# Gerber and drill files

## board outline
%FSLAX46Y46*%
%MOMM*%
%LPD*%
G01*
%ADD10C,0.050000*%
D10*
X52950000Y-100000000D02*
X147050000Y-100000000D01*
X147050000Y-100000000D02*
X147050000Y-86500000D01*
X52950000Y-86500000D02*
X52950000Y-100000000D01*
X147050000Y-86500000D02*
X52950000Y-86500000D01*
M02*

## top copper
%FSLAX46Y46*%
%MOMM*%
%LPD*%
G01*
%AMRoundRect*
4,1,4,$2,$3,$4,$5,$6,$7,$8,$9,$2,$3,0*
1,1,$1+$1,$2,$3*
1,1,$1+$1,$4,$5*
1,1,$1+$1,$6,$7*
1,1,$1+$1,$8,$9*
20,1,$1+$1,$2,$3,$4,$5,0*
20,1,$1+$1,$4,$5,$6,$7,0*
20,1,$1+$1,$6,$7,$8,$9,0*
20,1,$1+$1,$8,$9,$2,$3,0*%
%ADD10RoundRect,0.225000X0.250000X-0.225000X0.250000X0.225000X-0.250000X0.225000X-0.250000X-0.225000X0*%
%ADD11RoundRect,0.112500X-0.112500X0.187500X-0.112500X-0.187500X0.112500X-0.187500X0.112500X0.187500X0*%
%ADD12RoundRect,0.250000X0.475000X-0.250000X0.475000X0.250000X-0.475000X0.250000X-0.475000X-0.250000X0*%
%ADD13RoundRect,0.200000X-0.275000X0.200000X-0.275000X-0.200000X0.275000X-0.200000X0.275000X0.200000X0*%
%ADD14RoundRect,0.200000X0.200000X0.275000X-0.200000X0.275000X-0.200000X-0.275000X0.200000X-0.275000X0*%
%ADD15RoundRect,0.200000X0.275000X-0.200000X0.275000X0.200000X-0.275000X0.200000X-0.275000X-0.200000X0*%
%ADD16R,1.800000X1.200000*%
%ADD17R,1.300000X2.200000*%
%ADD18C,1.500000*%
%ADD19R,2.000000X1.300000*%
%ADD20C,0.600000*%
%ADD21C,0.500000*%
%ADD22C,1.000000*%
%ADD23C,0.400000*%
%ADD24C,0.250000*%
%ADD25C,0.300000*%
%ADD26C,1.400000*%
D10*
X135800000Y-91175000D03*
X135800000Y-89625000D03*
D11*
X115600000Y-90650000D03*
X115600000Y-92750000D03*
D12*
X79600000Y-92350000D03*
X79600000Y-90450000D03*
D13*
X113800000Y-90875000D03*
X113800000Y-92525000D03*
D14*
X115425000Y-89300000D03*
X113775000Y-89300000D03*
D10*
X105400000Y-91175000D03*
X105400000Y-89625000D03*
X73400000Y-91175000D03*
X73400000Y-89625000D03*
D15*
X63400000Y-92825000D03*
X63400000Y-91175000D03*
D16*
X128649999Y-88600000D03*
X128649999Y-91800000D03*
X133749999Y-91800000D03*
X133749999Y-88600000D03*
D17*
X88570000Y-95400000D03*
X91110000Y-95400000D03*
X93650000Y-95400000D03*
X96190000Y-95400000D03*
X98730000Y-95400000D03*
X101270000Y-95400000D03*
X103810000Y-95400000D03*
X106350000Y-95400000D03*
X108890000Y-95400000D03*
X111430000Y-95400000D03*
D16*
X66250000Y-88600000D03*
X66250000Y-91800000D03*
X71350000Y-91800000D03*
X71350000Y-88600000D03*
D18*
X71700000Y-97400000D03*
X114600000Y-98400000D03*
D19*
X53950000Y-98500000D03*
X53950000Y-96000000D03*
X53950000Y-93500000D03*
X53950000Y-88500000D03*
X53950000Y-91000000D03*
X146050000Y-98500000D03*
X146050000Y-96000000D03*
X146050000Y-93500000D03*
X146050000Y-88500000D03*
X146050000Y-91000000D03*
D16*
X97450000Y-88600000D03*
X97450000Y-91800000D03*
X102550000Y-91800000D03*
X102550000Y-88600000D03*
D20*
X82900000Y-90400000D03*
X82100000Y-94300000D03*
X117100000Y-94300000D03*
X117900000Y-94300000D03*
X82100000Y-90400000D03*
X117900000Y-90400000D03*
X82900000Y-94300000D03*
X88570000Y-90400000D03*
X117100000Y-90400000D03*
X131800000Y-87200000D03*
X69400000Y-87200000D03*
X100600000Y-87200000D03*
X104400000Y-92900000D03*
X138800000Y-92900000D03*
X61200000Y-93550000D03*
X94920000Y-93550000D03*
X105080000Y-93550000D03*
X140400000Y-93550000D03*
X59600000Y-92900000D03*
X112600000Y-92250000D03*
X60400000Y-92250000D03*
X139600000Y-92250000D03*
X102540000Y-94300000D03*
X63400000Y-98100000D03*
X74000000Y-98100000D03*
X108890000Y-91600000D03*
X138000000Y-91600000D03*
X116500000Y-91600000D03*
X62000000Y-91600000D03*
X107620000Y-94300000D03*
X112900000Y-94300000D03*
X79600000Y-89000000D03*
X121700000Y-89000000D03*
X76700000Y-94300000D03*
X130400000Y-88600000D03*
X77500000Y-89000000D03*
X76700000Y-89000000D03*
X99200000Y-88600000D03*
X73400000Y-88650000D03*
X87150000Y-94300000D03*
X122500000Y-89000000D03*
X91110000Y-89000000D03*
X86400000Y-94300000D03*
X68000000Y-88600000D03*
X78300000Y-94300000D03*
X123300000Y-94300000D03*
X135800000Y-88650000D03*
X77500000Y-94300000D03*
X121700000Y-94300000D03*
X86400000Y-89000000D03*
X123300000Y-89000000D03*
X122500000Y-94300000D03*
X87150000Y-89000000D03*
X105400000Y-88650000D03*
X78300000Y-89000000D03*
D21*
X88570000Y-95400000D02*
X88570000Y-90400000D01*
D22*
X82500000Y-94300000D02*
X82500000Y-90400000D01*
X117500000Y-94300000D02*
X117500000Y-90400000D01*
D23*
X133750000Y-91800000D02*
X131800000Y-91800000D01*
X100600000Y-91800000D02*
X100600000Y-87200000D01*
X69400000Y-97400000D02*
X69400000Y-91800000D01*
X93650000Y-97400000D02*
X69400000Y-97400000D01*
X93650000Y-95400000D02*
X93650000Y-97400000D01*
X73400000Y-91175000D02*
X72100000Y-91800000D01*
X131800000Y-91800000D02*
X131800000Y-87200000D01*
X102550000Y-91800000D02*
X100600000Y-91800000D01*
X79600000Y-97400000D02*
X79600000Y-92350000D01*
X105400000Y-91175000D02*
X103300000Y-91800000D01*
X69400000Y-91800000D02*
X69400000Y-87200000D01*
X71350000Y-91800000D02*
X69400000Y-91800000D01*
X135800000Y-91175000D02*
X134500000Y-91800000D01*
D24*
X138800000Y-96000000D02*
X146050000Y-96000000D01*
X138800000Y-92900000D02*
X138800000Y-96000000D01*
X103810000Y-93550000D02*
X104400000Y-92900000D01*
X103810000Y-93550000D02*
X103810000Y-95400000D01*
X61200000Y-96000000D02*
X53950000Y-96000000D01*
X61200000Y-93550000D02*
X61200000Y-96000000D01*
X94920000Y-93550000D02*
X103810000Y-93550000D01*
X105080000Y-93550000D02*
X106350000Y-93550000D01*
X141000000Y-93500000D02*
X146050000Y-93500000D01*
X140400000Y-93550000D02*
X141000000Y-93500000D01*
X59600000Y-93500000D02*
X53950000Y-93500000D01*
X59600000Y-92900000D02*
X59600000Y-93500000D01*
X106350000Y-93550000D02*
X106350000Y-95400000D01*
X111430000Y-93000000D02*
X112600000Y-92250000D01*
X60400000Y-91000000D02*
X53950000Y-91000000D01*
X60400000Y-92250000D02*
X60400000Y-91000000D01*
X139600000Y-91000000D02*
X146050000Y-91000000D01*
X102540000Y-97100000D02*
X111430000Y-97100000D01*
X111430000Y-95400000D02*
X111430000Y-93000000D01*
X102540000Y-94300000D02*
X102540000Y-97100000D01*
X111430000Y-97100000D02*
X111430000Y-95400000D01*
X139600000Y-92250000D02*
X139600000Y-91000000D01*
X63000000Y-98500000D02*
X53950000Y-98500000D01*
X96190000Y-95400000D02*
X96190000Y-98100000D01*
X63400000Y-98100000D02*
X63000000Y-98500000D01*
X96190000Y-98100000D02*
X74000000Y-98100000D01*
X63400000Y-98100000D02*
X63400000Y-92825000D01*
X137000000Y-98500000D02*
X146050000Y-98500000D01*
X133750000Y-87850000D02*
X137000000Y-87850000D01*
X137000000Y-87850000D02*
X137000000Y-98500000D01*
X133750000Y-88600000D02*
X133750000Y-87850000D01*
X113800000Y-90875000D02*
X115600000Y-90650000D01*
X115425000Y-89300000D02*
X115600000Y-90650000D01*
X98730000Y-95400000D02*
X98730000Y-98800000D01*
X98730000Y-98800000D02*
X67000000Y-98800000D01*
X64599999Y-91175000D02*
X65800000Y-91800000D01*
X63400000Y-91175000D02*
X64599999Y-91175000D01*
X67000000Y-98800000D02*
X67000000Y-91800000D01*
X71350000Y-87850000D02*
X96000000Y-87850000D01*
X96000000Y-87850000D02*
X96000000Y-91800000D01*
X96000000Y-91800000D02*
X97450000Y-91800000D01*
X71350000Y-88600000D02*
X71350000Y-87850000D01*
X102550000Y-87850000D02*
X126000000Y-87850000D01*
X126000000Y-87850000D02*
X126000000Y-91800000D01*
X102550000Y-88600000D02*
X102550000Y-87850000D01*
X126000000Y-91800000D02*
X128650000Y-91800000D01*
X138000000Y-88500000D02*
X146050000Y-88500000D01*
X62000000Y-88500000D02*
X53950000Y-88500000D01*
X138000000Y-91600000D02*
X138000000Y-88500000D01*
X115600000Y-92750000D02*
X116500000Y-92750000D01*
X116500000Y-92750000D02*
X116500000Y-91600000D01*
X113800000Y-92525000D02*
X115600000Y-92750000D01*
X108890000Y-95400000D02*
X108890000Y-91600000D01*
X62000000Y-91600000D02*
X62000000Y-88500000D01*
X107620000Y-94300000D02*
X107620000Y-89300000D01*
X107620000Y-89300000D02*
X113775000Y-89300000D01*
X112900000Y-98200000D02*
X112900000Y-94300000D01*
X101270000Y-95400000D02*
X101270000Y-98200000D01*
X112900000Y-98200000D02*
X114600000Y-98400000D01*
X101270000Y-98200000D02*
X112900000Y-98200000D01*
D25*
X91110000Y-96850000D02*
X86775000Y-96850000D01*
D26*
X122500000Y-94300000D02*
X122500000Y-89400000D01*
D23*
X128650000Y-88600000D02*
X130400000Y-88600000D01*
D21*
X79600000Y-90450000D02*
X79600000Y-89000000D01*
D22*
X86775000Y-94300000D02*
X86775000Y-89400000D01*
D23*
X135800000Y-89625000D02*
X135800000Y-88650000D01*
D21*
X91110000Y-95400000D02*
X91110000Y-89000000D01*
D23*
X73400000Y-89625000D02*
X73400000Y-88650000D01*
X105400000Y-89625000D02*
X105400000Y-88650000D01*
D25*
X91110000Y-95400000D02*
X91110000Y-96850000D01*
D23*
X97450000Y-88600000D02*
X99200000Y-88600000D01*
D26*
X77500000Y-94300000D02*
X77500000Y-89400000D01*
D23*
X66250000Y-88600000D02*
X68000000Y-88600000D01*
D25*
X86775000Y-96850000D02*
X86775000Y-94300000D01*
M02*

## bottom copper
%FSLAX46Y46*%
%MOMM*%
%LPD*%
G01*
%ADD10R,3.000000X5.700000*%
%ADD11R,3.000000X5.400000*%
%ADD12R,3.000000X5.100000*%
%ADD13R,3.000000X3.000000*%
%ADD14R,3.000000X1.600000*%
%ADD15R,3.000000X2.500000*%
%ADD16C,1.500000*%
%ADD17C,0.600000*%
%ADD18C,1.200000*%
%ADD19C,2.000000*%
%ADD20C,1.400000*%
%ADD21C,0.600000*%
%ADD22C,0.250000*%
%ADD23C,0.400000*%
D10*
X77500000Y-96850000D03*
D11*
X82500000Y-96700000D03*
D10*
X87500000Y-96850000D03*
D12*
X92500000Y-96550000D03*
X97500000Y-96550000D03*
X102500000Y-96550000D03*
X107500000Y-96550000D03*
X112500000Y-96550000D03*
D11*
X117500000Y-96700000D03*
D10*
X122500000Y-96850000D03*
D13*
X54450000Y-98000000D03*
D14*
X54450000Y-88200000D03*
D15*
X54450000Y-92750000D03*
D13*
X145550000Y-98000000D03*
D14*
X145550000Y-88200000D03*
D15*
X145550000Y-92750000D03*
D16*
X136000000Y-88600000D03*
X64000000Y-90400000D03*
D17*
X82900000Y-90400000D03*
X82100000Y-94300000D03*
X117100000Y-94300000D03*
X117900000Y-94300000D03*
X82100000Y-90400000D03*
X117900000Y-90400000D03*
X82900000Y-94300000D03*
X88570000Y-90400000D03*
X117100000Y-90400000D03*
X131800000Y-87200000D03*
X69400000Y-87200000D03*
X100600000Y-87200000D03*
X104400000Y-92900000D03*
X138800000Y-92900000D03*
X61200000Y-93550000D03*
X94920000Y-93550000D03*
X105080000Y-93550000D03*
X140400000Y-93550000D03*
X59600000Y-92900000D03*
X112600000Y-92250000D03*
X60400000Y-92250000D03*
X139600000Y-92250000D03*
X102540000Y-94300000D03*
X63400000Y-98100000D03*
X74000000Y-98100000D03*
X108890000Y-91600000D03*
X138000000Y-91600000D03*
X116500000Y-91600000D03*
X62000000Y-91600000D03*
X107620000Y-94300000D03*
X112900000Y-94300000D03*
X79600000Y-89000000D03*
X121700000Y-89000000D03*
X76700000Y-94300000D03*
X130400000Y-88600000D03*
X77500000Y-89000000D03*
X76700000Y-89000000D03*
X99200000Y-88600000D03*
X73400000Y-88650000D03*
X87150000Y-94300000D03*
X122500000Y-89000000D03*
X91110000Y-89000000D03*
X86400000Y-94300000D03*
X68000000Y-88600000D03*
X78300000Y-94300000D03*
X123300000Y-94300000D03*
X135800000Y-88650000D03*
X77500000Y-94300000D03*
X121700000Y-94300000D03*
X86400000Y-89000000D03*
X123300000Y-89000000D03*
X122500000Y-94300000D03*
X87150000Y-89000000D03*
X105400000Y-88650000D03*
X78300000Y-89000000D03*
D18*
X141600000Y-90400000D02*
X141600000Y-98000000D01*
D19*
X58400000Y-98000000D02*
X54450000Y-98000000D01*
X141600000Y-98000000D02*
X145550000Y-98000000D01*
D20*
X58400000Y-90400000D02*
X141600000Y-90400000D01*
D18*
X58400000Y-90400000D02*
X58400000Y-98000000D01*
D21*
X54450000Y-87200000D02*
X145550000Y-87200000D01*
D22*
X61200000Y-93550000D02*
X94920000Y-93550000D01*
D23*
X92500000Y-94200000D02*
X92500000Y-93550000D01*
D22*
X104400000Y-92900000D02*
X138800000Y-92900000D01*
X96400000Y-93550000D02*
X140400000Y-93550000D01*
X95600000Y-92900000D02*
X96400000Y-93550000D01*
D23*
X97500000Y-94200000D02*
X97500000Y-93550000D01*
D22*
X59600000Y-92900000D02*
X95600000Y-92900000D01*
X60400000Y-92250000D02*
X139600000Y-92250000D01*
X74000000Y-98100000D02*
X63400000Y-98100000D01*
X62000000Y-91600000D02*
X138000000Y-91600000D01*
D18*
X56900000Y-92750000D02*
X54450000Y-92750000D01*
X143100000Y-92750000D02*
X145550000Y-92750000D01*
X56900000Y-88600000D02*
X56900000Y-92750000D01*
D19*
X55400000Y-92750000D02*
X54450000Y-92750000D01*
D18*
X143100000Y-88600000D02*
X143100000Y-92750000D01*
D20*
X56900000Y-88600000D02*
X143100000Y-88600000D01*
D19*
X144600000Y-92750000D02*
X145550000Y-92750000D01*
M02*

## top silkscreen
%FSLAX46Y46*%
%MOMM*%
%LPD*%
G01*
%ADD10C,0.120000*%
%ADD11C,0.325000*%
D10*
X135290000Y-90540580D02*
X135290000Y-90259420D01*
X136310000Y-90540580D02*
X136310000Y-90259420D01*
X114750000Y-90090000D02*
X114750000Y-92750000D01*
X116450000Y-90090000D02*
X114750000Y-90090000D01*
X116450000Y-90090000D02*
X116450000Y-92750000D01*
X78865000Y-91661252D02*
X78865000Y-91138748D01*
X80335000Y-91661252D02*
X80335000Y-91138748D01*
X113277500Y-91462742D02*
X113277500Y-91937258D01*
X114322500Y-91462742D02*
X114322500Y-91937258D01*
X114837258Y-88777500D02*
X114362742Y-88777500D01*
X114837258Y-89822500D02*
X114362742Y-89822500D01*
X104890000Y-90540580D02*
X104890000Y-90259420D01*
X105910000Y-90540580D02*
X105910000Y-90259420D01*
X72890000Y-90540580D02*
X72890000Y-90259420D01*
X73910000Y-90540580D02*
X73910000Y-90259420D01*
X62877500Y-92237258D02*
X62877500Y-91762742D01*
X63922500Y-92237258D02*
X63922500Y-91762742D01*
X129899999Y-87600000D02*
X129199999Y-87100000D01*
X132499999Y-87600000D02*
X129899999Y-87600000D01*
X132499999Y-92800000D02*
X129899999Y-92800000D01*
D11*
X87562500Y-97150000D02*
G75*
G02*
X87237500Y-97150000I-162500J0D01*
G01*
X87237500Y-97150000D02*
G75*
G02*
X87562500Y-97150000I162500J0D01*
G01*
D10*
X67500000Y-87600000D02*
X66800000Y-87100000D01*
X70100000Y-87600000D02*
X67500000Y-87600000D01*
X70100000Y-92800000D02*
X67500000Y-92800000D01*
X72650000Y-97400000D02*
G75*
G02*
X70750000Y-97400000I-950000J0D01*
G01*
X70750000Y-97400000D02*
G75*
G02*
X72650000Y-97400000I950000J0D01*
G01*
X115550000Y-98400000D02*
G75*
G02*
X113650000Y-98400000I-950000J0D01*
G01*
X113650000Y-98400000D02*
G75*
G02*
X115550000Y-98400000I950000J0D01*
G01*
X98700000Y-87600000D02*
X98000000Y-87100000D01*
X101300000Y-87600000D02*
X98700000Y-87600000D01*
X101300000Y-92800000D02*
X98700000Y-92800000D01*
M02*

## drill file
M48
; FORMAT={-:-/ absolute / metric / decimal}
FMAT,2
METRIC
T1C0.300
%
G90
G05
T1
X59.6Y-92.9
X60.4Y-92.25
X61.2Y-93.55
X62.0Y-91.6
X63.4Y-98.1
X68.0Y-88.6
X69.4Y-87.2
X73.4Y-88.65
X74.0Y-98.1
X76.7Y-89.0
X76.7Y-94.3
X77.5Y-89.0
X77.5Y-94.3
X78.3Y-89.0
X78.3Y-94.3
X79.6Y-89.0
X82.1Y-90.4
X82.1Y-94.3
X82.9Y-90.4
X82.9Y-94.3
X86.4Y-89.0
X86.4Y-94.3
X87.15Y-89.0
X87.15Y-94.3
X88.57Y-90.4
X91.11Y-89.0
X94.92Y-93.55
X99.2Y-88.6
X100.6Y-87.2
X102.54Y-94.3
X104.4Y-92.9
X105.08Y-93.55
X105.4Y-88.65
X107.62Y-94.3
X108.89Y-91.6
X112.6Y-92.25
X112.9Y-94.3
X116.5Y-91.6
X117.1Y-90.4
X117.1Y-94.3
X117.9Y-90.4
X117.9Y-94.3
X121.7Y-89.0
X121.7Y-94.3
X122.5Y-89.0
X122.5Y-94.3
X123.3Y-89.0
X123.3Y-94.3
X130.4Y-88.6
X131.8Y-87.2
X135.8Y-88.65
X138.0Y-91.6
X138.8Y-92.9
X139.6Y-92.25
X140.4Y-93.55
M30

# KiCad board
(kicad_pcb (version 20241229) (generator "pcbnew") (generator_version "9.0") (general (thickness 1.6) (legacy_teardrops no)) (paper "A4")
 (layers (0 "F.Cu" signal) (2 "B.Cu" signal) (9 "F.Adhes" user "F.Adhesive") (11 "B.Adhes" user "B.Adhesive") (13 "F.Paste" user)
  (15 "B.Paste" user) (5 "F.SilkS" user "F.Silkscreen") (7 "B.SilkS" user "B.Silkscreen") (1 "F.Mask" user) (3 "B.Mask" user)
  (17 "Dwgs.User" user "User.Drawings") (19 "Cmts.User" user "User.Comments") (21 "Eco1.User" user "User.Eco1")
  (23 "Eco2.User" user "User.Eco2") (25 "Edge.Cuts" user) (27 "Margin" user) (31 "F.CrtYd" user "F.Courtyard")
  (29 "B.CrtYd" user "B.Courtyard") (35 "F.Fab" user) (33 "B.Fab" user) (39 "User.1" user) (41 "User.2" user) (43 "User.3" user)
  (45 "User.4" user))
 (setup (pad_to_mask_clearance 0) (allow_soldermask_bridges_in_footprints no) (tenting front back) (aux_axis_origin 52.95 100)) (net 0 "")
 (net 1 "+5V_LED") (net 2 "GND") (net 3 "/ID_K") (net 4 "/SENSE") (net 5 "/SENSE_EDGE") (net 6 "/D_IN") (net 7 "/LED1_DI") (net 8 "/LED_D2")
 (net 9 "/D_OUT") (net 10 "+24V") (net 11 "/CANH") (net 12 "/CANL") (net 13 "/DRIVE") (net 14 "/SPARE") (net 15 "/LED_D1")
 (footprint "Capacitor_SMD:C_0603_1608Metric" (layer "F.Cu") (at 135.8 90.4 90)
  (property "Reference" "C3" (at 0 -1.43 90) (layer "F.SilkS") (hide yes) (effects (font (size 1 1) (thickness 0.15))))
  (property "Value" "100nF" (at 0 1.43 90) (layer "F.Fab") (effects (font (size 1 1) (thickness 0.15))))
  (fp_line (start -0.14058 -0.51) (end 0.14058 -0.51) (stroke (width 0.12) (type solid)) (layer "F.SilkS"))
  (fp_line (start -0.14058 0.51) (end 0.14058 0.51) (stroke (width 0.12) (type solid)) (layer "F.SilkS"))
  (pad "1" smd roundrect (at -0.775 0 90) (size 0.9 0.95) (layers "F.Cu" "F.Mask" "F.Paste") (roundrect_rratio 0.25) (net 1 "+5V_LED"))
  (pad "2" smd roundrect (at 0.775 0 90) (size 0.9 0.95) (layers "F.Cu" "F.Mask" "F.Paste") (roundrect_rratio 0.25) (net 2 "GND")))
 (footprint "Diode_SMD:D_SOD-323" (layer "F.Cu") (at 115.6 91.7 -90)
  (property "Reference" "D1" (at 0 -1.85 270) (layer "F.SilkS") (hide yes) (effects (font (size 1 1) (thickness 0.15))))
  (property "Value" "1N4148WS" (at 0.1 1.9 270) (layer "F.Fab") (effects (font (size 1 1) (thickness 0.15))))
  (fp_line (start -1.61 0.85) (end 1.05 0.85) (stroke (width 0.12) (type solid)) (layer "F.SilkS"))
  (fp_line (start -1.61 -0.85) (end -1.61 0.85) (stroke (width 0.12) (type solid)) (layer "F.SilkS"))
  (fp_line (start -1.61 -0.85) (end 1.05 -0.85) (stroke (width 0.12) (type solid)) (layer "F.SilkS"))
  (pad "1" smd roundrect (at -1.05 0 270) (size 0.6 0.45) (layers "F.Cu" "F.Mask" "F.Paste") (roundrect_rratio 0.25) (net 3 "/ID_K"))
  (pad "2" smd roundrect (at 1.05 0 270) (size 0.6 0.45) (layers "F.Cu" "F.Mask" "F.Paste") (roundrect_rratio 0.25) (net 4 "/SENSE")))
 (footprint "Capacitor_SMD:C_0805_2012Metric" (layer "F.Cu") (at 79.6 91.4 90)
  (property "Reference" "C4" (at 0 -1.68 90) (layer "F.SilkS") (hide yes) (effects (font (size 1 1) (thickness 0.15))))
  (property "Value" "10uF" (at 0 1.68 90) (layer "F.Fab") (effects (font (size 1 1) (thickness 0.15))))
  (fp_line (start -0.261252 -0.735) (end 0.261252 -0.735) (stroke (width 0.12) (type solid)) (layer "F.SilkS"))
  (fp_line (start -0.261252 0.735) (end 0.261252 0.735) (stroke (width 0.12) (type solid)) (layer "F.SilkS"))
  (pad "1" smd roundrect (at -0.95 0 90) (size 1 1.45) (layers "F.Cu" "F.Mask" "F.Paste") (roundrect_rratio 0.25) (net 1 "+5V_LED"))
  (pad "2" smd roundrect (at 0.95 0 90) (size 1 1.45) (layers "F.Cu" "F.Mask" "F.Paste") (roundrect_rratio 0.25) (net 2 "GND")))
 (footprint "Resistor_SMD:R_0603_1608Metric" (layer "F.Cu") (at 113.8 91.7 -90)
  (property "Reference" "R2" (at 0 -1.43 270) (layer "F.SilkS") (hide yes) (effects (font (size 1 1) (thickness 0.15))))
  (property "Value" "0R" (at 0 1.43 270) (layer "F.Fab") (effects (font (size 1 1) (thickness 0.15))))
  (fp_line (start -0.237258 0.5225) (end 0.237258 0.5225) (stroke (width 0.12) (type solid)) (layer "F.SilkS"))
  (fp_line (start -0.237258 -0.5225) (end 0.237258 -0.5225) (stroke (width 0.12) (type solid)) (layer "F.SilkS"))
  (pad "1" smd roundrect (at -0.825 0 270) (size 0.8 0.95) (layers "F.Cu" "F.Mask" "F.Paste") (roundrect_rratio 0.25) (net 3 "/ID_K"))
  (pad "2" smd roundrect (at 0.825 0 270) (size 0.8 0.95) (layers "F.Cu" "F.Mask" "F.Paste") (roundrect_rratio 0.25) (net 4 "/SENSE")))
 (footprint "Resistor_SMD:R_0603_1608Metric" (layer "F.Cu") (at 114.6 89.3 180)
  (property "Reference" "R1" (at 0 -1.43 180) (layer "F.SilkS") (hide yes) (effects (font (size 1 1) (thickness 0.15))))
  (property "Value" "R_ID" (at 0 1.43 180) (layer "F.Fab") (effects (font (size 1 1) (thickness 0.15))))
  (fp_line (start -0.237258 0.5225) (end 0.237258 0.5225) (stroke (width 0.12) (type solid)) (layer "F.SilkS"))
  (fp_line (start -0.237258 -0.5225) (end 0.237258 -0.5225) (stroke (width 0.12) (type solid)) (layer "F.SilkS"))
  (pad "1" smd roundrect (at -0.825 0 180) (size 0.8 0.95) (layers "F.Cu" "F.Mask" "F.Paste") (roundrect_rratio 0.25) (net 3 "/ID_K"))
  (pad "2" smd roundrect (at 0.825 0 180) (size 0.8 0.95) (layers "F.Cu" "F.Mask" "F.Paste") (roundrect_rratio 0.25) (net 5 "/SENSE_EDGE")))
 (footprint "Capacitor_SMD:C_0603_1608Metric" (layer "F.Cu") (at 105.4 90.4 90)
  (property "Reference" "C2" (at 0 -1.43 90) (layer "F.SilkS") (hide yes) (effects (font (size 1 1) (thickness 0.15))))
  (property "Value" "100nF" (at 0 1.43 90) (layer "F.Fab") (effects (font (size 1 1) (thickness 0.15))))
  (fp_line (start -0.14058 -0.51) (end 0.14058 -0.51) (stroke (width 0.12) (type solid)) (layer "F.SilkS"))
  (fp_line (start -0.14058 0.51) (end 0.14058 0.51) (stroke (width 0.12) (type solid)) (layer "F.SilkS"))
  (pad "1" smd roundrect (at -0.775 0 90) (size 0.9 0.95) (layers "F.Cu" "F.Mask" "F.Paste") (roundrect_rratio 0.25) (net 1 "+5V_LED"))
  (pad "2" smd roundrect (at 0.775 0 90) (size 0.9 0.95) (layers "F.Cu" "F.Mask" "F.Paste") (roundrect_rratio 0.25) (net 2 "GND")))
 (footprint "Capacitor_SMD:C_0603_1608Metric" (layer "F.Cu") (at 73.4 90.4 90)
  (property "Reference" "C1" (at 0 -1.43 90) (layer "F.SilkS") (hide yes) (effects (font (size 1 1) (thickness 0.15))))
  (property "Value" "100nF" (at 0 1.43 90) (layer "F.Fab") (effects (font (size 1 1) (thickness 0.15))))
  (fp_line (start -0.14058 -0.51) (end 0.14058 -0.51) (stroke (width 0.12) (type solid)) (layer "F.SilkS"))
  (fp_line (start -0.14058 0.51) (end 0.14058 0.51) (stroke (width 0.12) (type solid)) (layer "F.SilkS"))
  (pad "1" smd roundrect (at -0.775 0 90) (size 0.9 0.95) (layers "F.Cu" "F.Mask" "F.Paste") (roundrect_rratio 0.25) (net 1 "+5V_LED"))
  (pad "2" smd roundrect (at 0.775 0 90) (size 0.9 0.95) (layers "F.Cu" "F.Mask" "F.Paste") (roundrect_rratio 0.25) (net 2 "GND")))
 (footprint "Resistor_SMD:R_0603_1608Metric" (layer "F.Cu") (at 63.4 92 90)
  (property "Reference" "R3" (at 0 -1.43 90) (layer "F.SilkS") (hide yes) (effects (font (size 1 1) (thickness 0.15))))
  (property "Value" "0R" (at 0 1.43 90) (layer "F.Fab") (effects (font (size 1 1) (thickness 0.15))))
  (fp_line (start -0.237258 -0.5225) (end 0.237258 -0.5225) (stroke (width 0.12) (type solid)) (layer "F.SilkS"))
  (fp_line (start -0.237258 0.5225) (end 0.237258 0.5225) (stroke (width 0.12) (type solid)) (layer "F.SilkS"))
  (pad "1" smd roundrect (at -0.825 0 90) (size 0.8 0.95) (layers "F.Cu" "F.Mask" "F.Paste") (roundrect_rratio 0.25) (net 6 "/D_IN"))
  (pad "2" smd roundrect (at 0.825 0 90) (size 0.8 0.95) (layers "F.Cu" "F.Mask" "F.Paste") (roundrect_rratio 0.25) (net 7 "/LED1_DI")))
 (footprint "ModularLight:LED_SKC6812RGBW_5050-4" (layer "F.Cu") (at 131.199999 90.2 180)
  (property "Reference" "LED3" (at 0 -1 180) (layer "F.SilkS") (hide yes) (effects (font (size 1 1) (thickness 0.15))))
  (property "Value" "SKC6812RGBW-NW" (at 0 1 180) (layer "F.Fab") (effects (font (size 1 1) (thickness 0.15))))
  (fp_line (start 1.3 2.6) (end 2 3.1) (stroke (width 0.12) (type solid)) (layer "F.SilkS"))
  (fp_line (start -1.3 2.6) (end 1.3 2.6) (stroke (width 0.12) (type solid)) (layer "F.SilkS"))
  (fp_line (start -1.3 -2.6) (end 1.3 -2.6) (stroke (width 0.12) (type solid)) (layer "F.SilkS"))
  (pad "1" smd rect (at 2.55 1.6 180) (size 1.8 1.2) (layers "F.Cu" "F.Mask" "F.Paste") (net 2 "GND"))
  (pad "2" smd rect (at 2.55 -1.6 180) (size 1.8 1.2) (layers "F.Cu" "F.Mask" "F.Paste") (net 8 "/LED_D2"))
  (pad "3" smd rect (at -2.55 -1.6 180) (size 1.8 1.2) (layers "F.Cu" "F.Mask" "F.Paste") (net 1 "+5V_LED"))
  (pad "4" smd rect (at -2.55 1.6 180) (size 1.8 1.2) (layers "F.Cu" "F.Mask" "F.Paste") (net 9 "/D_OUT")))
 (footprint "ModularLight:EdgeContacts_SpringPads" (layer "F.Cu") (at 100 100)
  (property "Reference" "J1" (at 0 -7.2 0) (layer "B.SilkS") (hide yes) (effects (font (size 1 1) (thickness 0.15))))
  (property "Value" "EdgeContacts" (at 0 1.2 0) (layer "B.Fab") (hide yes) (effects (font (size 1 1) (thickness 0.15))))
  (pad "X1" smd rect (at -22.5 -3.15) (size 3 5.7) (layers "B.Cu" "B.Mask") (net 2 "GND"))
  (pad "X2" smd rect (at -17.5 -3.3) (size 3 5.4) (layers "B.Cu" "B.Mask") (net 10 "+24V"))
  (pad "X3" smd rect (at -12.5 -3.15) (size 3 5.7) (layers "B.Cu" "B.Mask") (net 2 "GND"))
  (pad "X4" smd rect (at -7.5 -3.45) (size 3 5.1) (layers "B.Cu" "B.Mask") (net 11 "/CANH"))
  (pad "X5" smd rect (at -2.5 -3.45) (size 3 5.1) (layers "B.Cu" "B.Mask") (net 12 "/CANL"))
  (pad "X6" smd rect (at 2.5 -3.45) (size 3 5.1) (layers "B.Cu" "B.Mask") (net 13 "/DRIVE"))
  (pad "X7" smd rect (at 7.5 -3.45) (size 3 5.1) (layers "B.Cu" "B.Mask") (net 5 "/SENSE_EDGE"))
  (pad "X8" smd rect (at 12.5 -3.45) (size 3 5.1) (layers "B.Cu" "B.Mask") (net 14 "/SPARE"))
  (pad "X9" smd rect (at 17.5 -3.3) (size 3 5.4) (layers "B.Cu" "B.Mask") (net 10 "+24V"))
  (pad "X10" smd rect (at 22.5 -3.15) (size 3 5.7) (layers "B.Cu" "B.Mask") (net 2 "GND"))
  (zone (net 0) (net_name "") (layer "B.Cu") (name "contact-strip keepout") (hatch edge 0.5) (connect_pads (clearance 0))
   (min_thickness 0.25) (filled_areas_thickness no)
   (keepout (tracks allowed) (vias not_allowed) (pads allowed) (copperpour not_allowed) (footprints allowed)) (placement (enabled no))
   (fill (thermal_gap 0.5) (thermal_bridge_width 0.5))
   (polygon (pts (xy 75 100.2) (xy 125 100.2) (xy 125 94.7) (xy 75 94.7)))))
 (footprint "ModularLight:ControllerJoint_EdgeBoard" (layer "F.Cu") (at 100 94.75)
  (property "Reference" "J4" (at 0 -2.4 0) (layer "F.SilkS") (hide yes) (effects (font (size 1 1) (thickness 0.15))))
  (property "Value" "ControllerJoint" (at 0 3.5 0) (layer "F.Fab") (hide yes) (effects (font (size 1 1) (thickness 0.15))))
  (fp_circle (center -12.6 2.4) (end -12.35 2.4) (stroke (width 0.15) (type solid)) (fill yes) (layer "F.SilkS"))
  (pad "1" smd rect (at -11.43 0.65) (size 1.3 2.2) (layers "F.Cu" "F.Mask" "F.Paste") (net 10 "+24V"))
  (pad "2" smd rect (at -8.89 0.65) (size 1.3 2.2) (layers "F.Cu" "F.Mask" "F.Paste") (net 2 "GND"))
  (pad "3" smd rect (at -6.35 0.65) (size 1.3 2.2) (layers "F.Cu" "F.Mask" "F.Paste") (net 1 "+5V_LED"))
  (pad "4" smd rect (at -3.81 0.65) (size 1.3 2.2) (layers "F.Cu" "F.Mask" "F.Paste") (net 6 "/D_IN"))
  (pad "5" smd rect (at -1.27 0.65) (size 1.3 2.2) (layers "F.Cu" "F.Mask" "F.Paste") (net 7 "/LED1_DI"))
  (pad "6" smd rect (at 1.27 0.65) (size 1.3 2.2) (layers "F.Cu" "F.Mask" "F.Paste") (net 14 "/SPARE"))
  (pad "7" smd rect (at 3.81 0.65) (size 1.3 2.2) (layers "F.Cu" "F.Mask" "F.Paste") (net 11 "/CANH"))
  (pad "8" smd rect (at 6.35 0.65) (size 1.3 2.2) (layers "F.Cu" "F.Mask" "F.Paste") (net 12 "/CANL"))
  (pad "9" smd rect (at 8.89 0.65) (size 1.3 2.2) (layers "F.Cu" "F.Mask" "F.Paste") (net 4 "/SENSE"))
  (pad "10" smd rect (at 11.43 0.65) (size 1.3 2.2) (layers "F.Cu" "F.Mask" "F.Paste") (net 13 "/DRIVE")))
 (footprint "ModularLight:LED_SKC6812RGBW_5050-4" (layer "F.Cu") (at 68.8 90.2 180)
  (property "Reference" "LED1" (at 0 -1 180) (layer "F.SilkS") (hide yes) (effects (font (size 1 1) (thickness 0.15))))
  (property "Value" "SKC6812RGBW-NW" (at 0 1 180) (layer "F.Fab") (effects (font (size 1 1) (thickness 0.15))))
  (fp_line (start 1.3 2.6) (end 2 3.1) (stroke (width 0.12) (type solid)) (layer "F.SilkS"))
  (fp_line (start -1.3 2.6) (end 1.3 2.6) (stroke (width 0.12) (type solid)) (layer "F.SilkS"))
  (fp_line (start -1.3 -2.6) (end 1.3 -2.6) (stroke (width 0.12) (type solid)) (layer "F.SilkS"))
  (pad "1" smd rect (at 2.55 1.6 180) (size 1.8 1.2) (layers "F.Cu" "F.Mask" "F.Paste") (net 2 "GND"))
  (pad "2" smd rect (at 2.55 -1.6 180) (size 1.8 1.2) (layers "F.Cu" "F.Mask" "F.Paste") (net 7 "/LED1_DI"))
  (pad "3" smd rect (at -2.55 -1.6 180) (size 1.8 1.2) (layers "F.Cu" "F.Mask" "F.Paste") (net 1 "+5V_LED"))
  (pad "4" smd rect (at -2.55 1.6 180) (size 1.8 1.2) (layers "F.Cu" "F.Mask" "F.Paste") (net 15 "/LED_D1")))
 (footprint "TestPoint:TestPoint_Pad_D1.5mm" (layer "F.Cu") (at 71.7 97.4)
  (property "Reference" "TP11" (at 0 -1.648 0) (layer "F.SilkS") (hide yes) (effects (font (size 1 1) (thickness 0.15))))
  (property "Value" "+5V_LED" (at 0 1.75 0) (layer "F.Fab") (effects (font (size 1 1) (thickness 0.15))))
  (fp_circle (center 0 0) (end 0 0.95) (stroke (width 0.12) (type solid)) (fill no) (layer "F.SilkS"))
  (pad "1" smd circle (at 0 0) (size 1.5 1.5) (layers "F.Cu" "F.Mask") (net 1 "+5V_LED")))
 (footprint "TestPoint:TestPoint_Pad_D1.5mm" (layer "F.Cu") (at 114.6 98.4)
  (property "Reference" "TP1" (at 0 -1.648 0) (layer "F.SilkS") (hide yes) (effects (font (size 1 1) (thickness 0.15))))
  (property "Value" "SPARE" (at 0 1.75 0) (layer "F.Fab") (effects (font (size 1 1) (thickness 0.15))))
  (fp_circle (center 0 0) (end 0 0.95) (stroke (width 0.12) (type solid)) (fill no) (layer "F.SilkS"))
  (pad "1" smd circle (at 0 0) (size 1.5 1.5) (layers "F.Cu" "F.Mask") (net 14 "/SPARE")))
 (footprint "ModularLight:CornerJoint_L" (layer "F.Cu") (at 52.95 100)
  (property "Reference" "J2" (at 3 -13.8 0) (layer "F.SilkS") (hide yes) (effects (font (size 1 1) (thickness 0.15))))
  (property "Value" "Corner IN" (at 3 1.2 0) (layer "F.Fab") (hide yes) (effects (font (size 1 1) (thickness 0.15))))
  (pad "1" smd rect (at 1 -1.5) (size 2 1.3) (layers "F.Cu" "F.Mask" "F.Paste") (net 6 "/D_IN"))
  (pad "2" smd rect (at 1 -4) (size 2 1.3) (layers "F.Cu" "F.Mask" "F.Paste") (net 11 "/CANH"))
  (pad "3" smd rect (at 1 -6.5) (size 2 1.3) (layers "F.Cu" "F.Mask" "F.Paste") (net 12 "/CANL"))
  (pad "4" smd rect (at 1 -11.5) (size 2 1.3) (layers "F.Cu" "F.Mask" "F.Paste") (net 4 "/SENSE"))
  (pad "5" smd rect (at 1 -9) (size 2 1.3) (layers "F.Cu" "F.Mask" "F.Paste") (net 13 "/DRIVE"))
  (pad "6" smd rect (at 1.5 -2) (size 3 3) (layers "B.Cu" "B.Mask") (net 10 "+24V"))
  (pad "7" smd rect (at 1.5 -11.8) (size 3 1.6) (layers "B.Cu" "B.Mask") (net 1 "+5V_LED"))
  (pad "8" smd rect (at 1.5 -7.25) (size 3 2.5) (layers "B.Cu" "B.Mask") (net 2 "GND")))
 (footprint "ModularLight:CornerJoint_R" (layer "F.Cu") (at 147.05 100)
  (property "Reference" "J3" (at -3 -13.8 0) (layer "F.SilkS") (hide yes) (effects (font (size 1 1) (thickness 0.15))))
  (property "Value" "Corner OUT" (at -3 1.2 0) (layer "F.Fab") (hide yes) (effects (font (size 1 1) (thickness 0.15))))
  (pad "1" smd rect (at -1 -1.5) (size 2 1.3) (layers "F.Cu" "F.Mask" "F.Paste") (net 9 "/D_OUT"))
  (pad "2" smd rect (at -1 -4) (size 2 1.3) (layers "F.Cu" "F.Mask" "F.Paste") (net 11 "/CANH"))
  (pad "3" smd rect (at -1 -6.5) (size 2 1.3) (layers "F.Cu" "F.Mask" "F.Paste") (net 12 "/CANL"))
  (pad "4" smd rect (at -1 -11.5) (size 2 1.3) (layers "F.Cu" "F.Mask" "F.Paste") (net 4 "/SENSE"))
  (pad "5" smd rect (at -1 -9) (size 2 1.3) (layers "F.Cu" "F.Mask" "F.Paste") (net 13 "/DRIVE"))
  (pad "6" smd rect (at -1.5 -2) (size 3 3) (layers "B.Cu" "B.Mask") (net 10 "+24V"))
  (pad "7" smd rect (at -1.5 -11.8) (size 3 1.6) (layers "B.Cu" "B.Mask") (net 1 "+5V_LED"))
  (pad "8" smd rect (at -1.5 -7.25) (size 3 2.5) (layers "B.Cu" "B.Mask") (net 2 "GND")))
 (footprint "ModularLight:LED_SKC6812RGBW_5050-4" (layer "F.Cu") (at 100 90.2 180)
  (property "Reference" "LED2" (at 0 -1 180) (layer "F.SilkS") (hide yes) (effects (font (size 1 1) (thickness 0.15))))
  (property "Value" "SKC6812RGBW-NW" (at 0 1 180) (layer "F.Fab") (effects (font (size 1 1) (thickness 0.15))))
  (fp_line (start 1.3 2.6) (end 2 3.1) (stroke (width 0.12) (type solid)) (layer "F.SilkS"))
  (fp_line (start -1.3 2.6) (end 1.3 2.6) (stroke (width 0.12) (type solid)) (layer "F.SilkS"))
  (fp_line (start -1.3 -2.6) (end 1.3 -2.6) (stroke (width 0.12) (type solid)) (layer "F.SilkS"))
  (pad "1" smd rect (at 2.55 1.6 180) (size 1.8 1.2) (layers "F.Cu" "F.Mask" "F.Paste") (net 2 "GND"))
  (pad "2" smd rect (at 2.55 -1.6 180) (size 1.8 1.2) (layers "F.Cu" "F.Mask" "F.Paste") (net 15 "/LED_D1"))
  (pad "3" smd rect (at -2.55 -1.6 180) (size 1.8 1.2) (layers "F.Cu" "F.Mask" "F.Paste") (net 1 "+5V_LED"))
  (pad "4" smd rect (at -2.55 1.6 180) (size 1.8 1.2) (layers "F.Cu" "F.Mask" "F.Paste") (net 8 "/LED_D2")))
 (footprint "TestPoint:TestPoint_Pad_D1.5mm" (layer "B.Cu") (at 136 88.6 180)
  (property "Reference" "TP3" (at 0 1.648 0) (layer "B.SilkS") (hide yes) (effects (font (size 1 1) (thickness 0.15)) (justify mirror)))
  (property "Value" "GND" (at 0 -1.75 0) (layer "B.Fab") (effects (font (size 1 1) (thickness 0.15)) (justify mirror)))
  (pad "1" smd circle (at 0 0 180) (size 1.5 1.5) (layers "B.Cu" "B.Mask") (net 2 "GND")))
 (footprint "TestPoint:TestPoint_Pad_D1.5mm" (layer "B.Cu") (at 64 90.4 180)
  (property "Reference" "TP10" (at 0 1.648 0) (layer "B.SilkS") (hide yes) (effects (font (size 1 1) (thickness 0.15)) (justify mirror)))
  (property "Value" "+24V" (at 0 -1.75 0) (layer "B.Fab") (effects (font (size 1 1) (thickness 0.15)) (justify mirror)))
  (pad "1" smd circle (at 0 0 180) (size 1.5 1.5) (layers "B.Cu" "B.Mask") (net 10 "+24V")))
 (gr_line (start 52.95 100) (end 147.05 100) (stroke (width 0.05) (type default)) (layer "Edge.Cuts"))
 (gr_line (start 147.05 100) (end 147.05 86.5) (stroke (width 0.05) (type default)) (layer "Edge.Cuts"))
 (gr_line (start 52.95 86.5) (end 52.95 100) (stroke (width 0.05) (type default)) (layer "Edge.Cuts"))
 (gr_line (start 147.05 86.5) (end 52.95 86.5) (stroke (width 0.05) (type default)) (layer "Edge.Cuts"))
 (segment (start 88.57 95.4) (end 88.57 90.4) (width 0.5) (locked yes) (layer "F.Cu") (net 10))
 (segment (start 82.5 94.3) (end 82.5 90.4) (width 1) (locked yes) (layer "F.Cu") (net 10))
 (segment (start 117.5 94.3) (end 117.5 90.4) (width 1) (locked yes) (layer "F.Cu") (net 10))
 (via (at 82.9 90.4) (size 0.6) (drill 0.3) (layers "F.Cu" "B.Cu") (locked yes) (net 10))
 (via (at 82.1 94.3) (size 0.6) (drill 0.3) (layers "F.Cu" "B.Cu") (locked yes) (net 10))
 (via (at 117.1 94.3) (size 0.6) (drill 0.3) (layers "F.Cu" "B.Cu") (locked yes) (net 10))
 (via (at 117.9 94.3) (size 0.6) (drill 0.3) (layers "F.Cu" "B.Cu") (locked yes) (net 10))
 (via (at 82.1 90.4) (size 0.6) (drill 0.3) (layers "F.Cu" "B.Cu") (locked yes) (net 10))
 (via (at 117.9 90.4) (size 0.6) (drill 0.3) (layers "F.Cu" "B.Cu") (locked yes) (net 10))
 (via (at 82.9 94.3) (size 0.6) (drill 0.3) (layers "F.Cu" "B.Cu") (locked yes) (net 10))
 (via (at 88.57 90.4) (size 0.6) (drill 0.3) (layers "F.Cu" "B.Cu") (locked yes) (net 10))
 (via (at 117.1 90.4) (size 0.6) (drill 0.3) (layers "F.Cu" "B.Cu") (locked yes) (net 10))
 (segment (start 141.6 90.4) (end 141.6 98) (width 1.2) (locked yes) (layer "B.Cu") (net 10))
 (segment (start 58.4 98) (end 54.45 98) (width 2) (locked yes) (layer "B.Cu") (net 10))
 (segment (start 141.6 98) (end 145.55 98) (width 2) (locked yes) (layer "B.Cu") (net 10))
 (segment (start 58.4 90.4) (end 141.6 90.4) (width 1.4) (locked yes) (layer "B.Cu") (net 10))
 (segment (start 58.4 90.4) (end 58.4 98) (width 1.2) (locked yes) (layer "B.Cu") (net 10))
 (segment (start 133.75 91.8) (end 131.8 91.8) (width 0.4) (locked yes) (layer "F.Cu") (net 1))
 (segment (start 100.6 91.8) (end 100.6 87.2) (width 0.4) (locked yes) (layer "F.Cu") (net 1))
 (segment (start 69.4 97.4) (end 69.4 91.8) (width 0.4) (locked yes) (layer "F.Cu") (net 1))
 (segment (start 93.65 97.4) (end 69.4 97.4) (width 0.4) (locked yes) (layer "F.Cu") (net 1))
 (segment (start 93.65 95.4) (end 93.65 97.4) (width 0.4) (locked yes) (layer "F.Cu") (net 1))
 (segment (start 73.4 91.175) (end 72.1 91.8) (width 0.4) (locked yes) (layer "F.Cu") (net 1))
 (segment (start 131.8 91.8) (end 131.8 87.2) (width 0.4) (locked yes) (layer "F.Cu") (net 1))
 (segment (start 102.55 91.8) (end 100.6 91.8) (width 0.4) (locked yes) (layer "F.Cu") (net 1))
 (segment (start 79.6 97.4) (end 79.6 92.35) (width 0.4) (locked yes) (layer "F.Cu") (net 1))
 (segment (start 105.4 91.175) (end 103.3 91.8) (width 0.4) (locked yes) (layer "F.Cu") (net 1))
 (segment (start 69.4 91.8) (end 69.4 87.2) (width 0.4) (locked yes) (layer "F.Cu") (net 1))
 (segment (start 71.35 91.8) (end 69.4 91.8) (width 0.4) (locked yes) (layer "F.Cu") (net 1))
 (segment (start 135.8 91.175) (end 134.5 91.8) (width 0.4) (locked yes) (layer "F.Cu") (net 1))
 (via (at 131.8 87.2) (size 0.6) (drill 0.3) (layers "F.Cu" "B.Cu") (locked yes) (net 1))
 (via (at 69.4 87.2) (size 0.6) (drill 0.3) (layers "F.Cu" "B.Cu") (locked yes) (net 1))
 (via (at 100.6 87.2) (size 0.6) (drill 0.3) (layers "F.Cu" "B.Cu") (locked yes) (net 1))
 (segment (start 54.45 87.2) (end 145.55 87.2) (width 0.6) (locked yes) (layer "B.Cu") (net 1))
 (segment (start 138.8 96) (end 146.05 96) (width 0.25) (locked yes) (layer "F.Cu") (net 11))
 (segment (start 138.8 92.9) (end 138.8 96) (width 0.25) (locked yes) (layer "F.Cu") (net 11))
 (segment (start 103.81 93.55) (end 104.4 92.9) (width 0.25) (locked yes) (layer "F.Cu") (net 11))
 (segment (start 103.81 93.55) (end 103.81 95.4) (width 0.25) (locked yes) (layer "F.Cu") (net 11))
 (segment (start 61.2 96) (end 53.95 96) (width 0.25) (locked yes) (layer "F.Cu") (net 11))
 (segment (start 61.2 93.55) (end 61.2 96) (width 0.25) (locked yes) (layer "F.Cu") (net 11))
 (segment (start 94.92 93.55) (end 103.81 93.55) (width 0.25) (locked yes) (layer "F.Cu") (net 11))
 (via (at 104.4 92.9) (size 0.6) (drill 0.3) (layers "F.Cu" "B.Cu") (locked yes) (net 11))
 (via (at 138.8 92.9) (size 0.6) (drill 0.3) (layers "F.Cu" "B.Cu") (locked yes) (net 11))
 (via (at 61.2 93.55) (size 0.6) (drill 0.3) (layers "F.Cu" "B.Cu") (locked yes) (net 11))
 (via (at 94.92 93.55) (size 0.6) (drill 0.3) (layers "F.Cu" "B.Cu") (locked yes) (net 11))
 (segment (start 61.2 93.55) (end 94.92 93.55) (width 0.25) (locked yes) (layer "B.Cu") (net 11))
 (segment (start 92.5 94.2) (end 92.5 93.55) (width 0.4) (locked yes) (layer "B.Cu") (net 11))
 (segment (start 104.4 92.9) (end 138.8 92.9) (width 0.25) (locked yes) (layer "B.Cu") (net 11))
 (segment (start 105.08 93.55) (end 106.35 93.55) (width 0.25) (locked yes) (layer "F.Cu") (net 12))
 (segment (start 141 93.5) (end 146.05 93.5) (width 0.25) (locked yes) (layer "F.Cu") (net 12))
 (segment (start 140.4 93.55) (end 141 93.5) (width 0.25) (locked yes) (layer "F.Cu") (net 12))
 (segment (start 59.6 93.5) (end 53.95 93.5) (width 0.25) (locked yes) (layer "F.Cu") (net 12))
 (segment (start 59.6 92.9) (end 59.6 93.5) (width 0.25) (locked yes) (layer "F.Cu") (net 12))
 (segment (start 106.35 93.55) (end 106.35 95.4) (width 0.25) (locked yes) (layer "F.Cu") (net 12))
 (via (at 105.08 93.55) (size 0.6) (drill 0.3) (layers "F.Cu" "B.Cu") (locked yes) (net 12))
 (via (at 140.4 93.55) (size 0.6) (drill 0.3) (layers "F.Cu" "B.Cu") (locked yes) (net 12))
 (via (at 59.6 92.9) (size 0.6) (drill 0.3) (layers "F.Cu" "B.Cu") (locked yes) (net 12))
 (segment (start 96.4 93.55) (end 140.4 93.55) (width 0.25) (locked yes) (layer "B.Cu") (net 12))
 (segment (start 95.6 92.9) (end 96.4 93.55) (width 0.25) (locked yes) (layer "B.Cu") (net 12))
 (segment (start 97.5 94.2) (end 97.5 93.55) (width 0.4) (locked yes) (layer "B.Cu") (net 12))
 (segment (start 59.6 92.9) (end 95.6 92.9) (width 0.25) (locked yes) (layer "B.Cu") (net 12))
 (segment (start 111.43 93) (end 112.6 92.25) (width 0.25) (locked yes) (layer "F.Cu") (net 13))
 (segment (start 60.4 91) (end 53.95 91) (width 0.25) (locked yes) (layer "F.Cu") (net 13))
 (segment (start 60.4 92.25) (end 60.4 91) (width 0.25) (locked yes) (layer "F.Cu") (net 13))
 (segment (start 139.6 91) (end 146.05 91) (width 0.25) (locked yes) (layer "F.Cu") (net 13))
 (segment (start 102.54 97.1) (end 111.43 97.1) (width 0.25) (locked yes) (layer "F.Cu") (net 13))
 (segment (start 111.43 95.4) (end 111.43 93) (width 0.25) (locked yes) (layer "F.Cu") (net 13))
 (segment (start 102.54 94.3) (end 102.54 97.1) (width 0.25) (locked yes) (layer "F.Cu") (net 13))
 (segment (start 111.43 97.1) (end 111.43 95.4) (width 0.25) (locked yes) (layer "F.Cu") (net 13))
 (segment (start 139.6 92.25) (end 139.6 91) (width 0.25) (locked yes) (layer "F.Cu") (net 13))
 (via (at 112.6 92.25) (size 0.6) (drill 0.3) (layers "F.Cu" "B.Cu") (locked yes) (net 13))
 (via (at 60.4 92.25) (size 0.6) (drill 0.3) (layers "F.Cu" "B.Cu") (locked yes) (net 13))
 (via (at 139.6 92.25) (size 0.6) (drill 0.3) (layers "F.Cu" "B.Cu") (locked yes) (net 13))
 (via (at 102.54 94.3) (size 0.6) (drill 0.3) (layers "F.Cu" "B.Cu") (locked yes) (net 13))
 (segment (start 60.4 92.25) (end 139.6 92.25) (width 0.25) (locked yes) (layer "B.Cu") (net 13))
 (segment (start 63 98.5) (end 53.95 98.5) (width 0.25) (locked yes) (layer "F.Cu") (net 6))
 (segment (start 96.19 95.4) (end 96.19 98.1) (width 0.25) (locked yes) (layer "F.Cu") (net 6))
 (segment (start 63.4 98.1) (end 63 98.5) (width 0.25) (locked yes) (layer "F.Cu") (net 6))
 (segment (start 96.19 98.1) (end 74 98.1) (width 0.25) (locked yes) (layer "F.Cu") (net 6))
 (segment (start 63.4 98.1) (end 63.4 92.825) (width 0.25) (locked yes) (layer "F.Cu") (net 6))
 (via (at 63.4 98.1) (size 0.6) (drill 0.3) (layers "F.Cu" "B.Cu") (locked yes) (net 6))
 (via (at 74 98.1) (size 0.6) (drill 0.3) (layers "F.Cu" "B.Cu") (locked yes) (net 6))
 (segment (start 74 98.1) (end 63.4 98.1) (width 0.25) (locked yes) (layer "B.Cu") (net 6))
 (segment (start 137 98.5) (end 146.05 98.5) (width 0.25) (locked yes) (layer "F.Cu") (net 9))
 (segment (start 133.75 87.85) (end 137 87.85) (width 0.25) (locked yes) (layer "F.Cu") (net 9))
 (segment (start 137 87.85) (end 137 98.5) (width 0.25) (locked yes) (layer "F.Cu") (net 9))
 (segment (start 133.75 88.6) (end 133.75 87.85) (width 0.25) (locked yes) (layer "F.Cu") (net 9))
 (segment (start 113.8 90.875) (end 115.6 90.65) (width 0.25) (locked yes) (layer "F.Cu") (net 3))
 (segment (start 115.425 89.3) (end 115.6 90.65) (width 0.25) (locked yes) (layer "F.Cu") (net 3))
 (segment (start 98.73 95.4) (end 98.73 98.8) (width 0.25) (locked yes) (layer "F.Cu") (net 7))
 (segment (start 98.73 98.8) (end 67 98.8) (width 0.25) (locked yes) (layer "F.Cu") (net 7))
 (segment (start 64.599999 91.175) (end 65.8 91.8) (width 0.25) (locked yes) (layer "F.Cu") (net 7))
 (segment (start 63.4 91.175) (end 64.599999 91.175) (width 0.25) (locked yes) (layer "F.Cu") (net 7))
 (segment (start 67 98.8) (end 67 91.8) (width 0.25) (locked yes) (layer "F.Cu") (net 7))
 (segment (start 71.35 87.85) (end 96 87.85) (width 0.25) (locked yes) (layer "F.Cu") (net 15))
 (segment (start 96 87.85) (end 96 91.8) (width 0.25) (locked yes) (layer "F.Cu") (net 15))
 (segment (start 96 91.8) (end 97.45 91.8) (width 0.25) (locked yes) (layer "F.Cu") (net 15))
 (segment (start 71.35 88.6) (end 71.35 87.85) (width 0.25) (locked yes) (layer "F.Cu") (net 15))
 (segment (start 102.55 87.85) (end 126 87.85) (width 0.25) (locked yes) (layer "F.Cu") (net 8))
 (segment (start 126 87.85) (end 126 91.8) (width 0.25) (locked yes) (layer "F.Cu") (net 8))
 (segment (start 102.55 88.6) (end 102.55 87.85) (width 0.25) (locked yes) (layer "F.Cu") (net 8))
 (segment (start 126 91.8) (end 128.65 91.8) (width 0.25) (locked yes) (layer "F.Cu") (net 8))
 (segment (start 138 88.5) (end 146.05 88.5) (width 0.25) (locked yes) (layer "F.Cu") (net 4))
 (segment (start 62 88.5) (end 53.95 88.5) (width 0.25) (locked yes) (layer "F.Cu") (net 4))
 (segment (start 138 91.6) (end 138 88.5) (width 0.25) (locked yes) (layer "F.Cu") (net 4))
 (segment (start 115.6 92.75) (end 116.5 92.75) (width 0.25) (locked yes) (layer "F.Cu") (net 4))
 (segment (start 116.5 92.75) (end 116.5 91.6) (width 0.25) (locked yes) (layer "F.Cu") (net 4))
 (segment (start 113.8 92.525) (end 115.6 92.75) (width 0.25) (locked yes) (layer "F.Cu") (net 4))
 (segment (start 108.89 95.4) (end 108.89 91.6) (width 0.25) (locked yes) (layer "F.Cu") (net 4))
 (segment (start 62 91.6) (end 62 88.5) (width 0.25) (locked yes) (layer "F.Cu") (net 4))
 (via (at 108.89 91.6) (size 0.6) (drill 0.3) (layers "F.Cu" "B.Cu") (locked yes) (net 4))
 (via (at 138 91.6) (size 0.6) (drill 0.3) (layers "F.Cu" "B.Cu") (locked yes) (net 4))
 (via (at 116.5 91.6) (size 0.6) (drill 0.3) (layers "F.Cu" "B.Cu") (locked yes) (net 4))
 (via (at 62 91.6) (size 0.6) (drill 0.3) (layers "F.Cu" "B.Cu") (locked yes) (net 4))
 (segment (start 62 91.6) (end 138 91.6) (width 0.25) (locked yes) (layer "B.Cu") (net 4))
 (segment (start 107.62 94.3) (end 107.62 89.3) (width 0.25) (locked yes) (layer "F.Cu") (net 5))
 (segment (start 107.62 89.3) (end 113.775 89.3) (width 0.25) (locked yes) (layer "F.Cu") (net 5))
 (via (at 107.62 94.3) (size 0.6) (drill 0.3) (layers "F.Cu" "B.Cu") (locked yes) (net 5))
 (segment (start 112.9 98.2) (end 112.9 94.3) (width 0.25) (locked yes) (layer "F.Cu") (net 14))
 (segment (start 101.27 95.4) (end 101.27 98.2) (width 0.25) (locked yes) (layer "F.Cu") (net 14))
 (segment (start 112.9 98.2) (end 114.6 98.4) (width 0.25) (locked yes) (layer "F.Cu") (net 14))
 (segment (start 101.27 98.2) (end 112.9 98.2) (width 0.25) (locked yes) (layer "F.Cu") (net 14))
 (via (at 112.9 94.3) (size 0.6) (drill 0.3) (layers "F.Cu" "B.Cu") (locked yes) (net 14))
 (segment (start 91.11 96.85) (end 86.775 96.85) (width 0.3) (locked yes) (layer "F.Cu") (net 2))
 (segment (start 122.5 94.3) (end 122.5 89.4) (width 1.4) (locked yes) (layer "F.Cu") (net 2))
 (segment (start 128.65 88.6) (end 130.4 88.6) (width 0.4) (locked yes) (layer "F.Cu") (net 2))
 (segment (start 79.6 90.45) (end 79.6 89) (width 0.5) (locked yes) (layer "F.Cu") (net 2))
 (segment (start 86.775 94.3) (end 86.775 89.4) (width 1) (locked yes) (layer "F.Cu") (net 2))
 (segment (start 135.8 89.625) (end 135.8 88.65) (width 0.4) (locked yes) (layer "F.Cu") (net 2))
 (segment (start 91.11 95.4) (end 91.11 89) (width 0.5) (locked yes) (layer "F.Cu") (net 2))
 (segment (start 73.4 89.625) (end 73.4 88.65) (width 0.4) (locked yes) (layer "F.Cu") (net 2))
 (segment (start 105.4 89.625) (end 105.4 88.65) (width 0.4) (locked yes) (layer "F.Cu") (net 2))
 (segment (start 91.11 95.4) (end 91.11 96.85) (width 0.3) (locked yes) (layer "F.Cu") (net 2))
 (segment (start 97.45 88.6) (end 99.2 88.6) (width 0.4) (locked yes) (layer "F.Cu") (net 2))
 (segment (start 77.5 94.3) (end 77.5 89.4) (width 1.4) (locked yes) (layer "F.Cu") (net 2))
 (segment (start 66.25 88.6) (end 68 88.6) (width 0.4) (locked yes) (layer "F.Cu") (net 2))
 (segment (start 86.775 96.85) (end 86.775 94.3) (width 0.3) (locked yes) (layer "F.Cu") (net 2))
 (via (at 79.6 89) (size 0.6) (drill 0.3) (layers "F.Cu" "B.Cu") (locked yes) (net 2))
 (via (at 121.7 89) (size 0.6) (drill 0.3) (layers "F.Cu" "B.Cu") (locked yes) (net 2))
 (via (at 76.7 94.3) (size 0.6) (drill 0.3) (layers "F.Cu" "B.Cu") (locked yes) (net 2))
 (via (at 130.4 88.6) (size 0.6) (drill 0.3) (layers "F.Cu" "B.Cu") (locked yes) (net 2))
 (via (at 77.5 89) (size 0.6) (drill 0.3) (layers "F.Cu" "B.Cu") (locked yes) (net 2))
 (via (at 76.7 89) (size 0.6) (drill 0.3) (layers "F.Cu" "B.Cu") (locked yes) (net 2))
 (via (at 99.2 88.6) (size 0.6) (drill 0.3) (layers "F.Cu" "B.Cu") (locked yes) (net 2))
 (via (at 73.4 88.65) (size 0.6) (drill 0.3) (layers "F.Cu" "B.Cu") (locked yes) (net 2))
 (via (at 87.15 94.3) (size 0.6) (drill 0.3) (layers "F.Cu" "B.Cu") (locked yes) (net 2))
 (via (at 122.5 89) (size 0.6) (drill 0.3) (layers "F.Cu" "B.Cu") (locked yes) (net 2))
 (via (at 91.11 89) (size 0.6) (drill 0.3) (layers "F.Cu" "B.Cu") (locked yes) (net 2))
 (via (at 86.4 94.3) (size 0.6) (drill 0.3) (layers "F.Cu" "B.Cu") (locked yes) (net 2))
 (via (at 68 88.6) (size 0.6) (drill 0.3) (layers "F.Cu" "B.Cu") (locked yes) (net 2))
 (via (at 78.3 94.3) (size 0.6) (drill 0.3) (layers "F.Cu" "B.Cu") (locked yes) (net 2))
 (via (at 123.3 94.3) (size 0.6) (drill 0.3) (layers "F.Cu" "B.Cu") (locked yes) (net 2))
 (via (at 135.8 88.65) (size 0.6) (drill 0.3) (layers "F.Cu" "B.Cu") (locked yes) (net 2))
 (via (at 77.5 94.3) (size 0.6) (drill 0.3) (layers "F.Cu" "B.Cu") (locked yes) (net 2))
 (via (at 121.7 94.3) (size 0.6) (drill 0.3) (layers "F.Cu" "B.Cu") (locked yes) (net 2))
 (via (at 86.4 89) (size 0.6) (drill 0.3) (layers "F.Cu" "B.Cu") (locked yes) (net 2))
 (via (at 123.3 89) (size 0.6) (drill 0.3) (layers "F.Cu" "B.Cu") (locked yes) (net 2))
 (via (at 122.5 94.3) (size 0.6) (drill 0.3) (layers "F.Cu" "B.Cu") (locked yes) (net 2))
 (via (at 87.15 89) (size 0.6) (drill 0.3) (layers "F.Cu" "B.Cu") (locked yes) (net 2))
 (via (at 105.4 88.65) (size 0.6) (drill 0.3) (layers "F.Cu" "B.Cu") (locked yes) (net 2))
 (via (at 78.3 89) (size 0.6) (drill 0.3) (layers "F.Cu" "B.Cu") (locked yes) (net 2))
 (segment (start 56.9 92.75) (end 54.45 92.75) (width 1.2) (locked yes) (layer "B.Cu") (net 2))
 (segment (start 143.1 92.75) (end 145.55 92.75) (width 1.2) (locked yes) (layer "B.Cu") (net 2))
 (segment (start 56.9 88.6) (end 56.9 92.75) (width 1.2) (locked yes) (layer "B.Cu") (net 2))
 (segment (start 55.4 92.75) (end 54.45 92.75) (width 2) (locked yes) (layer "B.Cu") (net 2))
 (segment (start 143.1 88.6) (end 143.1 92.75) (width 1.2) (locked yes) (layer "B.Cu") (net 2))
 (segment (start 56.9 88.6) (end 143.1 88.6) (width 1.4) (locked yes) (layer "B.Cu") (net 2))
 (segment (start 144.6 92.75) (end 145.55 92.75) (width 2) (locked yes) (layer "B.Cu") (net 2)))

